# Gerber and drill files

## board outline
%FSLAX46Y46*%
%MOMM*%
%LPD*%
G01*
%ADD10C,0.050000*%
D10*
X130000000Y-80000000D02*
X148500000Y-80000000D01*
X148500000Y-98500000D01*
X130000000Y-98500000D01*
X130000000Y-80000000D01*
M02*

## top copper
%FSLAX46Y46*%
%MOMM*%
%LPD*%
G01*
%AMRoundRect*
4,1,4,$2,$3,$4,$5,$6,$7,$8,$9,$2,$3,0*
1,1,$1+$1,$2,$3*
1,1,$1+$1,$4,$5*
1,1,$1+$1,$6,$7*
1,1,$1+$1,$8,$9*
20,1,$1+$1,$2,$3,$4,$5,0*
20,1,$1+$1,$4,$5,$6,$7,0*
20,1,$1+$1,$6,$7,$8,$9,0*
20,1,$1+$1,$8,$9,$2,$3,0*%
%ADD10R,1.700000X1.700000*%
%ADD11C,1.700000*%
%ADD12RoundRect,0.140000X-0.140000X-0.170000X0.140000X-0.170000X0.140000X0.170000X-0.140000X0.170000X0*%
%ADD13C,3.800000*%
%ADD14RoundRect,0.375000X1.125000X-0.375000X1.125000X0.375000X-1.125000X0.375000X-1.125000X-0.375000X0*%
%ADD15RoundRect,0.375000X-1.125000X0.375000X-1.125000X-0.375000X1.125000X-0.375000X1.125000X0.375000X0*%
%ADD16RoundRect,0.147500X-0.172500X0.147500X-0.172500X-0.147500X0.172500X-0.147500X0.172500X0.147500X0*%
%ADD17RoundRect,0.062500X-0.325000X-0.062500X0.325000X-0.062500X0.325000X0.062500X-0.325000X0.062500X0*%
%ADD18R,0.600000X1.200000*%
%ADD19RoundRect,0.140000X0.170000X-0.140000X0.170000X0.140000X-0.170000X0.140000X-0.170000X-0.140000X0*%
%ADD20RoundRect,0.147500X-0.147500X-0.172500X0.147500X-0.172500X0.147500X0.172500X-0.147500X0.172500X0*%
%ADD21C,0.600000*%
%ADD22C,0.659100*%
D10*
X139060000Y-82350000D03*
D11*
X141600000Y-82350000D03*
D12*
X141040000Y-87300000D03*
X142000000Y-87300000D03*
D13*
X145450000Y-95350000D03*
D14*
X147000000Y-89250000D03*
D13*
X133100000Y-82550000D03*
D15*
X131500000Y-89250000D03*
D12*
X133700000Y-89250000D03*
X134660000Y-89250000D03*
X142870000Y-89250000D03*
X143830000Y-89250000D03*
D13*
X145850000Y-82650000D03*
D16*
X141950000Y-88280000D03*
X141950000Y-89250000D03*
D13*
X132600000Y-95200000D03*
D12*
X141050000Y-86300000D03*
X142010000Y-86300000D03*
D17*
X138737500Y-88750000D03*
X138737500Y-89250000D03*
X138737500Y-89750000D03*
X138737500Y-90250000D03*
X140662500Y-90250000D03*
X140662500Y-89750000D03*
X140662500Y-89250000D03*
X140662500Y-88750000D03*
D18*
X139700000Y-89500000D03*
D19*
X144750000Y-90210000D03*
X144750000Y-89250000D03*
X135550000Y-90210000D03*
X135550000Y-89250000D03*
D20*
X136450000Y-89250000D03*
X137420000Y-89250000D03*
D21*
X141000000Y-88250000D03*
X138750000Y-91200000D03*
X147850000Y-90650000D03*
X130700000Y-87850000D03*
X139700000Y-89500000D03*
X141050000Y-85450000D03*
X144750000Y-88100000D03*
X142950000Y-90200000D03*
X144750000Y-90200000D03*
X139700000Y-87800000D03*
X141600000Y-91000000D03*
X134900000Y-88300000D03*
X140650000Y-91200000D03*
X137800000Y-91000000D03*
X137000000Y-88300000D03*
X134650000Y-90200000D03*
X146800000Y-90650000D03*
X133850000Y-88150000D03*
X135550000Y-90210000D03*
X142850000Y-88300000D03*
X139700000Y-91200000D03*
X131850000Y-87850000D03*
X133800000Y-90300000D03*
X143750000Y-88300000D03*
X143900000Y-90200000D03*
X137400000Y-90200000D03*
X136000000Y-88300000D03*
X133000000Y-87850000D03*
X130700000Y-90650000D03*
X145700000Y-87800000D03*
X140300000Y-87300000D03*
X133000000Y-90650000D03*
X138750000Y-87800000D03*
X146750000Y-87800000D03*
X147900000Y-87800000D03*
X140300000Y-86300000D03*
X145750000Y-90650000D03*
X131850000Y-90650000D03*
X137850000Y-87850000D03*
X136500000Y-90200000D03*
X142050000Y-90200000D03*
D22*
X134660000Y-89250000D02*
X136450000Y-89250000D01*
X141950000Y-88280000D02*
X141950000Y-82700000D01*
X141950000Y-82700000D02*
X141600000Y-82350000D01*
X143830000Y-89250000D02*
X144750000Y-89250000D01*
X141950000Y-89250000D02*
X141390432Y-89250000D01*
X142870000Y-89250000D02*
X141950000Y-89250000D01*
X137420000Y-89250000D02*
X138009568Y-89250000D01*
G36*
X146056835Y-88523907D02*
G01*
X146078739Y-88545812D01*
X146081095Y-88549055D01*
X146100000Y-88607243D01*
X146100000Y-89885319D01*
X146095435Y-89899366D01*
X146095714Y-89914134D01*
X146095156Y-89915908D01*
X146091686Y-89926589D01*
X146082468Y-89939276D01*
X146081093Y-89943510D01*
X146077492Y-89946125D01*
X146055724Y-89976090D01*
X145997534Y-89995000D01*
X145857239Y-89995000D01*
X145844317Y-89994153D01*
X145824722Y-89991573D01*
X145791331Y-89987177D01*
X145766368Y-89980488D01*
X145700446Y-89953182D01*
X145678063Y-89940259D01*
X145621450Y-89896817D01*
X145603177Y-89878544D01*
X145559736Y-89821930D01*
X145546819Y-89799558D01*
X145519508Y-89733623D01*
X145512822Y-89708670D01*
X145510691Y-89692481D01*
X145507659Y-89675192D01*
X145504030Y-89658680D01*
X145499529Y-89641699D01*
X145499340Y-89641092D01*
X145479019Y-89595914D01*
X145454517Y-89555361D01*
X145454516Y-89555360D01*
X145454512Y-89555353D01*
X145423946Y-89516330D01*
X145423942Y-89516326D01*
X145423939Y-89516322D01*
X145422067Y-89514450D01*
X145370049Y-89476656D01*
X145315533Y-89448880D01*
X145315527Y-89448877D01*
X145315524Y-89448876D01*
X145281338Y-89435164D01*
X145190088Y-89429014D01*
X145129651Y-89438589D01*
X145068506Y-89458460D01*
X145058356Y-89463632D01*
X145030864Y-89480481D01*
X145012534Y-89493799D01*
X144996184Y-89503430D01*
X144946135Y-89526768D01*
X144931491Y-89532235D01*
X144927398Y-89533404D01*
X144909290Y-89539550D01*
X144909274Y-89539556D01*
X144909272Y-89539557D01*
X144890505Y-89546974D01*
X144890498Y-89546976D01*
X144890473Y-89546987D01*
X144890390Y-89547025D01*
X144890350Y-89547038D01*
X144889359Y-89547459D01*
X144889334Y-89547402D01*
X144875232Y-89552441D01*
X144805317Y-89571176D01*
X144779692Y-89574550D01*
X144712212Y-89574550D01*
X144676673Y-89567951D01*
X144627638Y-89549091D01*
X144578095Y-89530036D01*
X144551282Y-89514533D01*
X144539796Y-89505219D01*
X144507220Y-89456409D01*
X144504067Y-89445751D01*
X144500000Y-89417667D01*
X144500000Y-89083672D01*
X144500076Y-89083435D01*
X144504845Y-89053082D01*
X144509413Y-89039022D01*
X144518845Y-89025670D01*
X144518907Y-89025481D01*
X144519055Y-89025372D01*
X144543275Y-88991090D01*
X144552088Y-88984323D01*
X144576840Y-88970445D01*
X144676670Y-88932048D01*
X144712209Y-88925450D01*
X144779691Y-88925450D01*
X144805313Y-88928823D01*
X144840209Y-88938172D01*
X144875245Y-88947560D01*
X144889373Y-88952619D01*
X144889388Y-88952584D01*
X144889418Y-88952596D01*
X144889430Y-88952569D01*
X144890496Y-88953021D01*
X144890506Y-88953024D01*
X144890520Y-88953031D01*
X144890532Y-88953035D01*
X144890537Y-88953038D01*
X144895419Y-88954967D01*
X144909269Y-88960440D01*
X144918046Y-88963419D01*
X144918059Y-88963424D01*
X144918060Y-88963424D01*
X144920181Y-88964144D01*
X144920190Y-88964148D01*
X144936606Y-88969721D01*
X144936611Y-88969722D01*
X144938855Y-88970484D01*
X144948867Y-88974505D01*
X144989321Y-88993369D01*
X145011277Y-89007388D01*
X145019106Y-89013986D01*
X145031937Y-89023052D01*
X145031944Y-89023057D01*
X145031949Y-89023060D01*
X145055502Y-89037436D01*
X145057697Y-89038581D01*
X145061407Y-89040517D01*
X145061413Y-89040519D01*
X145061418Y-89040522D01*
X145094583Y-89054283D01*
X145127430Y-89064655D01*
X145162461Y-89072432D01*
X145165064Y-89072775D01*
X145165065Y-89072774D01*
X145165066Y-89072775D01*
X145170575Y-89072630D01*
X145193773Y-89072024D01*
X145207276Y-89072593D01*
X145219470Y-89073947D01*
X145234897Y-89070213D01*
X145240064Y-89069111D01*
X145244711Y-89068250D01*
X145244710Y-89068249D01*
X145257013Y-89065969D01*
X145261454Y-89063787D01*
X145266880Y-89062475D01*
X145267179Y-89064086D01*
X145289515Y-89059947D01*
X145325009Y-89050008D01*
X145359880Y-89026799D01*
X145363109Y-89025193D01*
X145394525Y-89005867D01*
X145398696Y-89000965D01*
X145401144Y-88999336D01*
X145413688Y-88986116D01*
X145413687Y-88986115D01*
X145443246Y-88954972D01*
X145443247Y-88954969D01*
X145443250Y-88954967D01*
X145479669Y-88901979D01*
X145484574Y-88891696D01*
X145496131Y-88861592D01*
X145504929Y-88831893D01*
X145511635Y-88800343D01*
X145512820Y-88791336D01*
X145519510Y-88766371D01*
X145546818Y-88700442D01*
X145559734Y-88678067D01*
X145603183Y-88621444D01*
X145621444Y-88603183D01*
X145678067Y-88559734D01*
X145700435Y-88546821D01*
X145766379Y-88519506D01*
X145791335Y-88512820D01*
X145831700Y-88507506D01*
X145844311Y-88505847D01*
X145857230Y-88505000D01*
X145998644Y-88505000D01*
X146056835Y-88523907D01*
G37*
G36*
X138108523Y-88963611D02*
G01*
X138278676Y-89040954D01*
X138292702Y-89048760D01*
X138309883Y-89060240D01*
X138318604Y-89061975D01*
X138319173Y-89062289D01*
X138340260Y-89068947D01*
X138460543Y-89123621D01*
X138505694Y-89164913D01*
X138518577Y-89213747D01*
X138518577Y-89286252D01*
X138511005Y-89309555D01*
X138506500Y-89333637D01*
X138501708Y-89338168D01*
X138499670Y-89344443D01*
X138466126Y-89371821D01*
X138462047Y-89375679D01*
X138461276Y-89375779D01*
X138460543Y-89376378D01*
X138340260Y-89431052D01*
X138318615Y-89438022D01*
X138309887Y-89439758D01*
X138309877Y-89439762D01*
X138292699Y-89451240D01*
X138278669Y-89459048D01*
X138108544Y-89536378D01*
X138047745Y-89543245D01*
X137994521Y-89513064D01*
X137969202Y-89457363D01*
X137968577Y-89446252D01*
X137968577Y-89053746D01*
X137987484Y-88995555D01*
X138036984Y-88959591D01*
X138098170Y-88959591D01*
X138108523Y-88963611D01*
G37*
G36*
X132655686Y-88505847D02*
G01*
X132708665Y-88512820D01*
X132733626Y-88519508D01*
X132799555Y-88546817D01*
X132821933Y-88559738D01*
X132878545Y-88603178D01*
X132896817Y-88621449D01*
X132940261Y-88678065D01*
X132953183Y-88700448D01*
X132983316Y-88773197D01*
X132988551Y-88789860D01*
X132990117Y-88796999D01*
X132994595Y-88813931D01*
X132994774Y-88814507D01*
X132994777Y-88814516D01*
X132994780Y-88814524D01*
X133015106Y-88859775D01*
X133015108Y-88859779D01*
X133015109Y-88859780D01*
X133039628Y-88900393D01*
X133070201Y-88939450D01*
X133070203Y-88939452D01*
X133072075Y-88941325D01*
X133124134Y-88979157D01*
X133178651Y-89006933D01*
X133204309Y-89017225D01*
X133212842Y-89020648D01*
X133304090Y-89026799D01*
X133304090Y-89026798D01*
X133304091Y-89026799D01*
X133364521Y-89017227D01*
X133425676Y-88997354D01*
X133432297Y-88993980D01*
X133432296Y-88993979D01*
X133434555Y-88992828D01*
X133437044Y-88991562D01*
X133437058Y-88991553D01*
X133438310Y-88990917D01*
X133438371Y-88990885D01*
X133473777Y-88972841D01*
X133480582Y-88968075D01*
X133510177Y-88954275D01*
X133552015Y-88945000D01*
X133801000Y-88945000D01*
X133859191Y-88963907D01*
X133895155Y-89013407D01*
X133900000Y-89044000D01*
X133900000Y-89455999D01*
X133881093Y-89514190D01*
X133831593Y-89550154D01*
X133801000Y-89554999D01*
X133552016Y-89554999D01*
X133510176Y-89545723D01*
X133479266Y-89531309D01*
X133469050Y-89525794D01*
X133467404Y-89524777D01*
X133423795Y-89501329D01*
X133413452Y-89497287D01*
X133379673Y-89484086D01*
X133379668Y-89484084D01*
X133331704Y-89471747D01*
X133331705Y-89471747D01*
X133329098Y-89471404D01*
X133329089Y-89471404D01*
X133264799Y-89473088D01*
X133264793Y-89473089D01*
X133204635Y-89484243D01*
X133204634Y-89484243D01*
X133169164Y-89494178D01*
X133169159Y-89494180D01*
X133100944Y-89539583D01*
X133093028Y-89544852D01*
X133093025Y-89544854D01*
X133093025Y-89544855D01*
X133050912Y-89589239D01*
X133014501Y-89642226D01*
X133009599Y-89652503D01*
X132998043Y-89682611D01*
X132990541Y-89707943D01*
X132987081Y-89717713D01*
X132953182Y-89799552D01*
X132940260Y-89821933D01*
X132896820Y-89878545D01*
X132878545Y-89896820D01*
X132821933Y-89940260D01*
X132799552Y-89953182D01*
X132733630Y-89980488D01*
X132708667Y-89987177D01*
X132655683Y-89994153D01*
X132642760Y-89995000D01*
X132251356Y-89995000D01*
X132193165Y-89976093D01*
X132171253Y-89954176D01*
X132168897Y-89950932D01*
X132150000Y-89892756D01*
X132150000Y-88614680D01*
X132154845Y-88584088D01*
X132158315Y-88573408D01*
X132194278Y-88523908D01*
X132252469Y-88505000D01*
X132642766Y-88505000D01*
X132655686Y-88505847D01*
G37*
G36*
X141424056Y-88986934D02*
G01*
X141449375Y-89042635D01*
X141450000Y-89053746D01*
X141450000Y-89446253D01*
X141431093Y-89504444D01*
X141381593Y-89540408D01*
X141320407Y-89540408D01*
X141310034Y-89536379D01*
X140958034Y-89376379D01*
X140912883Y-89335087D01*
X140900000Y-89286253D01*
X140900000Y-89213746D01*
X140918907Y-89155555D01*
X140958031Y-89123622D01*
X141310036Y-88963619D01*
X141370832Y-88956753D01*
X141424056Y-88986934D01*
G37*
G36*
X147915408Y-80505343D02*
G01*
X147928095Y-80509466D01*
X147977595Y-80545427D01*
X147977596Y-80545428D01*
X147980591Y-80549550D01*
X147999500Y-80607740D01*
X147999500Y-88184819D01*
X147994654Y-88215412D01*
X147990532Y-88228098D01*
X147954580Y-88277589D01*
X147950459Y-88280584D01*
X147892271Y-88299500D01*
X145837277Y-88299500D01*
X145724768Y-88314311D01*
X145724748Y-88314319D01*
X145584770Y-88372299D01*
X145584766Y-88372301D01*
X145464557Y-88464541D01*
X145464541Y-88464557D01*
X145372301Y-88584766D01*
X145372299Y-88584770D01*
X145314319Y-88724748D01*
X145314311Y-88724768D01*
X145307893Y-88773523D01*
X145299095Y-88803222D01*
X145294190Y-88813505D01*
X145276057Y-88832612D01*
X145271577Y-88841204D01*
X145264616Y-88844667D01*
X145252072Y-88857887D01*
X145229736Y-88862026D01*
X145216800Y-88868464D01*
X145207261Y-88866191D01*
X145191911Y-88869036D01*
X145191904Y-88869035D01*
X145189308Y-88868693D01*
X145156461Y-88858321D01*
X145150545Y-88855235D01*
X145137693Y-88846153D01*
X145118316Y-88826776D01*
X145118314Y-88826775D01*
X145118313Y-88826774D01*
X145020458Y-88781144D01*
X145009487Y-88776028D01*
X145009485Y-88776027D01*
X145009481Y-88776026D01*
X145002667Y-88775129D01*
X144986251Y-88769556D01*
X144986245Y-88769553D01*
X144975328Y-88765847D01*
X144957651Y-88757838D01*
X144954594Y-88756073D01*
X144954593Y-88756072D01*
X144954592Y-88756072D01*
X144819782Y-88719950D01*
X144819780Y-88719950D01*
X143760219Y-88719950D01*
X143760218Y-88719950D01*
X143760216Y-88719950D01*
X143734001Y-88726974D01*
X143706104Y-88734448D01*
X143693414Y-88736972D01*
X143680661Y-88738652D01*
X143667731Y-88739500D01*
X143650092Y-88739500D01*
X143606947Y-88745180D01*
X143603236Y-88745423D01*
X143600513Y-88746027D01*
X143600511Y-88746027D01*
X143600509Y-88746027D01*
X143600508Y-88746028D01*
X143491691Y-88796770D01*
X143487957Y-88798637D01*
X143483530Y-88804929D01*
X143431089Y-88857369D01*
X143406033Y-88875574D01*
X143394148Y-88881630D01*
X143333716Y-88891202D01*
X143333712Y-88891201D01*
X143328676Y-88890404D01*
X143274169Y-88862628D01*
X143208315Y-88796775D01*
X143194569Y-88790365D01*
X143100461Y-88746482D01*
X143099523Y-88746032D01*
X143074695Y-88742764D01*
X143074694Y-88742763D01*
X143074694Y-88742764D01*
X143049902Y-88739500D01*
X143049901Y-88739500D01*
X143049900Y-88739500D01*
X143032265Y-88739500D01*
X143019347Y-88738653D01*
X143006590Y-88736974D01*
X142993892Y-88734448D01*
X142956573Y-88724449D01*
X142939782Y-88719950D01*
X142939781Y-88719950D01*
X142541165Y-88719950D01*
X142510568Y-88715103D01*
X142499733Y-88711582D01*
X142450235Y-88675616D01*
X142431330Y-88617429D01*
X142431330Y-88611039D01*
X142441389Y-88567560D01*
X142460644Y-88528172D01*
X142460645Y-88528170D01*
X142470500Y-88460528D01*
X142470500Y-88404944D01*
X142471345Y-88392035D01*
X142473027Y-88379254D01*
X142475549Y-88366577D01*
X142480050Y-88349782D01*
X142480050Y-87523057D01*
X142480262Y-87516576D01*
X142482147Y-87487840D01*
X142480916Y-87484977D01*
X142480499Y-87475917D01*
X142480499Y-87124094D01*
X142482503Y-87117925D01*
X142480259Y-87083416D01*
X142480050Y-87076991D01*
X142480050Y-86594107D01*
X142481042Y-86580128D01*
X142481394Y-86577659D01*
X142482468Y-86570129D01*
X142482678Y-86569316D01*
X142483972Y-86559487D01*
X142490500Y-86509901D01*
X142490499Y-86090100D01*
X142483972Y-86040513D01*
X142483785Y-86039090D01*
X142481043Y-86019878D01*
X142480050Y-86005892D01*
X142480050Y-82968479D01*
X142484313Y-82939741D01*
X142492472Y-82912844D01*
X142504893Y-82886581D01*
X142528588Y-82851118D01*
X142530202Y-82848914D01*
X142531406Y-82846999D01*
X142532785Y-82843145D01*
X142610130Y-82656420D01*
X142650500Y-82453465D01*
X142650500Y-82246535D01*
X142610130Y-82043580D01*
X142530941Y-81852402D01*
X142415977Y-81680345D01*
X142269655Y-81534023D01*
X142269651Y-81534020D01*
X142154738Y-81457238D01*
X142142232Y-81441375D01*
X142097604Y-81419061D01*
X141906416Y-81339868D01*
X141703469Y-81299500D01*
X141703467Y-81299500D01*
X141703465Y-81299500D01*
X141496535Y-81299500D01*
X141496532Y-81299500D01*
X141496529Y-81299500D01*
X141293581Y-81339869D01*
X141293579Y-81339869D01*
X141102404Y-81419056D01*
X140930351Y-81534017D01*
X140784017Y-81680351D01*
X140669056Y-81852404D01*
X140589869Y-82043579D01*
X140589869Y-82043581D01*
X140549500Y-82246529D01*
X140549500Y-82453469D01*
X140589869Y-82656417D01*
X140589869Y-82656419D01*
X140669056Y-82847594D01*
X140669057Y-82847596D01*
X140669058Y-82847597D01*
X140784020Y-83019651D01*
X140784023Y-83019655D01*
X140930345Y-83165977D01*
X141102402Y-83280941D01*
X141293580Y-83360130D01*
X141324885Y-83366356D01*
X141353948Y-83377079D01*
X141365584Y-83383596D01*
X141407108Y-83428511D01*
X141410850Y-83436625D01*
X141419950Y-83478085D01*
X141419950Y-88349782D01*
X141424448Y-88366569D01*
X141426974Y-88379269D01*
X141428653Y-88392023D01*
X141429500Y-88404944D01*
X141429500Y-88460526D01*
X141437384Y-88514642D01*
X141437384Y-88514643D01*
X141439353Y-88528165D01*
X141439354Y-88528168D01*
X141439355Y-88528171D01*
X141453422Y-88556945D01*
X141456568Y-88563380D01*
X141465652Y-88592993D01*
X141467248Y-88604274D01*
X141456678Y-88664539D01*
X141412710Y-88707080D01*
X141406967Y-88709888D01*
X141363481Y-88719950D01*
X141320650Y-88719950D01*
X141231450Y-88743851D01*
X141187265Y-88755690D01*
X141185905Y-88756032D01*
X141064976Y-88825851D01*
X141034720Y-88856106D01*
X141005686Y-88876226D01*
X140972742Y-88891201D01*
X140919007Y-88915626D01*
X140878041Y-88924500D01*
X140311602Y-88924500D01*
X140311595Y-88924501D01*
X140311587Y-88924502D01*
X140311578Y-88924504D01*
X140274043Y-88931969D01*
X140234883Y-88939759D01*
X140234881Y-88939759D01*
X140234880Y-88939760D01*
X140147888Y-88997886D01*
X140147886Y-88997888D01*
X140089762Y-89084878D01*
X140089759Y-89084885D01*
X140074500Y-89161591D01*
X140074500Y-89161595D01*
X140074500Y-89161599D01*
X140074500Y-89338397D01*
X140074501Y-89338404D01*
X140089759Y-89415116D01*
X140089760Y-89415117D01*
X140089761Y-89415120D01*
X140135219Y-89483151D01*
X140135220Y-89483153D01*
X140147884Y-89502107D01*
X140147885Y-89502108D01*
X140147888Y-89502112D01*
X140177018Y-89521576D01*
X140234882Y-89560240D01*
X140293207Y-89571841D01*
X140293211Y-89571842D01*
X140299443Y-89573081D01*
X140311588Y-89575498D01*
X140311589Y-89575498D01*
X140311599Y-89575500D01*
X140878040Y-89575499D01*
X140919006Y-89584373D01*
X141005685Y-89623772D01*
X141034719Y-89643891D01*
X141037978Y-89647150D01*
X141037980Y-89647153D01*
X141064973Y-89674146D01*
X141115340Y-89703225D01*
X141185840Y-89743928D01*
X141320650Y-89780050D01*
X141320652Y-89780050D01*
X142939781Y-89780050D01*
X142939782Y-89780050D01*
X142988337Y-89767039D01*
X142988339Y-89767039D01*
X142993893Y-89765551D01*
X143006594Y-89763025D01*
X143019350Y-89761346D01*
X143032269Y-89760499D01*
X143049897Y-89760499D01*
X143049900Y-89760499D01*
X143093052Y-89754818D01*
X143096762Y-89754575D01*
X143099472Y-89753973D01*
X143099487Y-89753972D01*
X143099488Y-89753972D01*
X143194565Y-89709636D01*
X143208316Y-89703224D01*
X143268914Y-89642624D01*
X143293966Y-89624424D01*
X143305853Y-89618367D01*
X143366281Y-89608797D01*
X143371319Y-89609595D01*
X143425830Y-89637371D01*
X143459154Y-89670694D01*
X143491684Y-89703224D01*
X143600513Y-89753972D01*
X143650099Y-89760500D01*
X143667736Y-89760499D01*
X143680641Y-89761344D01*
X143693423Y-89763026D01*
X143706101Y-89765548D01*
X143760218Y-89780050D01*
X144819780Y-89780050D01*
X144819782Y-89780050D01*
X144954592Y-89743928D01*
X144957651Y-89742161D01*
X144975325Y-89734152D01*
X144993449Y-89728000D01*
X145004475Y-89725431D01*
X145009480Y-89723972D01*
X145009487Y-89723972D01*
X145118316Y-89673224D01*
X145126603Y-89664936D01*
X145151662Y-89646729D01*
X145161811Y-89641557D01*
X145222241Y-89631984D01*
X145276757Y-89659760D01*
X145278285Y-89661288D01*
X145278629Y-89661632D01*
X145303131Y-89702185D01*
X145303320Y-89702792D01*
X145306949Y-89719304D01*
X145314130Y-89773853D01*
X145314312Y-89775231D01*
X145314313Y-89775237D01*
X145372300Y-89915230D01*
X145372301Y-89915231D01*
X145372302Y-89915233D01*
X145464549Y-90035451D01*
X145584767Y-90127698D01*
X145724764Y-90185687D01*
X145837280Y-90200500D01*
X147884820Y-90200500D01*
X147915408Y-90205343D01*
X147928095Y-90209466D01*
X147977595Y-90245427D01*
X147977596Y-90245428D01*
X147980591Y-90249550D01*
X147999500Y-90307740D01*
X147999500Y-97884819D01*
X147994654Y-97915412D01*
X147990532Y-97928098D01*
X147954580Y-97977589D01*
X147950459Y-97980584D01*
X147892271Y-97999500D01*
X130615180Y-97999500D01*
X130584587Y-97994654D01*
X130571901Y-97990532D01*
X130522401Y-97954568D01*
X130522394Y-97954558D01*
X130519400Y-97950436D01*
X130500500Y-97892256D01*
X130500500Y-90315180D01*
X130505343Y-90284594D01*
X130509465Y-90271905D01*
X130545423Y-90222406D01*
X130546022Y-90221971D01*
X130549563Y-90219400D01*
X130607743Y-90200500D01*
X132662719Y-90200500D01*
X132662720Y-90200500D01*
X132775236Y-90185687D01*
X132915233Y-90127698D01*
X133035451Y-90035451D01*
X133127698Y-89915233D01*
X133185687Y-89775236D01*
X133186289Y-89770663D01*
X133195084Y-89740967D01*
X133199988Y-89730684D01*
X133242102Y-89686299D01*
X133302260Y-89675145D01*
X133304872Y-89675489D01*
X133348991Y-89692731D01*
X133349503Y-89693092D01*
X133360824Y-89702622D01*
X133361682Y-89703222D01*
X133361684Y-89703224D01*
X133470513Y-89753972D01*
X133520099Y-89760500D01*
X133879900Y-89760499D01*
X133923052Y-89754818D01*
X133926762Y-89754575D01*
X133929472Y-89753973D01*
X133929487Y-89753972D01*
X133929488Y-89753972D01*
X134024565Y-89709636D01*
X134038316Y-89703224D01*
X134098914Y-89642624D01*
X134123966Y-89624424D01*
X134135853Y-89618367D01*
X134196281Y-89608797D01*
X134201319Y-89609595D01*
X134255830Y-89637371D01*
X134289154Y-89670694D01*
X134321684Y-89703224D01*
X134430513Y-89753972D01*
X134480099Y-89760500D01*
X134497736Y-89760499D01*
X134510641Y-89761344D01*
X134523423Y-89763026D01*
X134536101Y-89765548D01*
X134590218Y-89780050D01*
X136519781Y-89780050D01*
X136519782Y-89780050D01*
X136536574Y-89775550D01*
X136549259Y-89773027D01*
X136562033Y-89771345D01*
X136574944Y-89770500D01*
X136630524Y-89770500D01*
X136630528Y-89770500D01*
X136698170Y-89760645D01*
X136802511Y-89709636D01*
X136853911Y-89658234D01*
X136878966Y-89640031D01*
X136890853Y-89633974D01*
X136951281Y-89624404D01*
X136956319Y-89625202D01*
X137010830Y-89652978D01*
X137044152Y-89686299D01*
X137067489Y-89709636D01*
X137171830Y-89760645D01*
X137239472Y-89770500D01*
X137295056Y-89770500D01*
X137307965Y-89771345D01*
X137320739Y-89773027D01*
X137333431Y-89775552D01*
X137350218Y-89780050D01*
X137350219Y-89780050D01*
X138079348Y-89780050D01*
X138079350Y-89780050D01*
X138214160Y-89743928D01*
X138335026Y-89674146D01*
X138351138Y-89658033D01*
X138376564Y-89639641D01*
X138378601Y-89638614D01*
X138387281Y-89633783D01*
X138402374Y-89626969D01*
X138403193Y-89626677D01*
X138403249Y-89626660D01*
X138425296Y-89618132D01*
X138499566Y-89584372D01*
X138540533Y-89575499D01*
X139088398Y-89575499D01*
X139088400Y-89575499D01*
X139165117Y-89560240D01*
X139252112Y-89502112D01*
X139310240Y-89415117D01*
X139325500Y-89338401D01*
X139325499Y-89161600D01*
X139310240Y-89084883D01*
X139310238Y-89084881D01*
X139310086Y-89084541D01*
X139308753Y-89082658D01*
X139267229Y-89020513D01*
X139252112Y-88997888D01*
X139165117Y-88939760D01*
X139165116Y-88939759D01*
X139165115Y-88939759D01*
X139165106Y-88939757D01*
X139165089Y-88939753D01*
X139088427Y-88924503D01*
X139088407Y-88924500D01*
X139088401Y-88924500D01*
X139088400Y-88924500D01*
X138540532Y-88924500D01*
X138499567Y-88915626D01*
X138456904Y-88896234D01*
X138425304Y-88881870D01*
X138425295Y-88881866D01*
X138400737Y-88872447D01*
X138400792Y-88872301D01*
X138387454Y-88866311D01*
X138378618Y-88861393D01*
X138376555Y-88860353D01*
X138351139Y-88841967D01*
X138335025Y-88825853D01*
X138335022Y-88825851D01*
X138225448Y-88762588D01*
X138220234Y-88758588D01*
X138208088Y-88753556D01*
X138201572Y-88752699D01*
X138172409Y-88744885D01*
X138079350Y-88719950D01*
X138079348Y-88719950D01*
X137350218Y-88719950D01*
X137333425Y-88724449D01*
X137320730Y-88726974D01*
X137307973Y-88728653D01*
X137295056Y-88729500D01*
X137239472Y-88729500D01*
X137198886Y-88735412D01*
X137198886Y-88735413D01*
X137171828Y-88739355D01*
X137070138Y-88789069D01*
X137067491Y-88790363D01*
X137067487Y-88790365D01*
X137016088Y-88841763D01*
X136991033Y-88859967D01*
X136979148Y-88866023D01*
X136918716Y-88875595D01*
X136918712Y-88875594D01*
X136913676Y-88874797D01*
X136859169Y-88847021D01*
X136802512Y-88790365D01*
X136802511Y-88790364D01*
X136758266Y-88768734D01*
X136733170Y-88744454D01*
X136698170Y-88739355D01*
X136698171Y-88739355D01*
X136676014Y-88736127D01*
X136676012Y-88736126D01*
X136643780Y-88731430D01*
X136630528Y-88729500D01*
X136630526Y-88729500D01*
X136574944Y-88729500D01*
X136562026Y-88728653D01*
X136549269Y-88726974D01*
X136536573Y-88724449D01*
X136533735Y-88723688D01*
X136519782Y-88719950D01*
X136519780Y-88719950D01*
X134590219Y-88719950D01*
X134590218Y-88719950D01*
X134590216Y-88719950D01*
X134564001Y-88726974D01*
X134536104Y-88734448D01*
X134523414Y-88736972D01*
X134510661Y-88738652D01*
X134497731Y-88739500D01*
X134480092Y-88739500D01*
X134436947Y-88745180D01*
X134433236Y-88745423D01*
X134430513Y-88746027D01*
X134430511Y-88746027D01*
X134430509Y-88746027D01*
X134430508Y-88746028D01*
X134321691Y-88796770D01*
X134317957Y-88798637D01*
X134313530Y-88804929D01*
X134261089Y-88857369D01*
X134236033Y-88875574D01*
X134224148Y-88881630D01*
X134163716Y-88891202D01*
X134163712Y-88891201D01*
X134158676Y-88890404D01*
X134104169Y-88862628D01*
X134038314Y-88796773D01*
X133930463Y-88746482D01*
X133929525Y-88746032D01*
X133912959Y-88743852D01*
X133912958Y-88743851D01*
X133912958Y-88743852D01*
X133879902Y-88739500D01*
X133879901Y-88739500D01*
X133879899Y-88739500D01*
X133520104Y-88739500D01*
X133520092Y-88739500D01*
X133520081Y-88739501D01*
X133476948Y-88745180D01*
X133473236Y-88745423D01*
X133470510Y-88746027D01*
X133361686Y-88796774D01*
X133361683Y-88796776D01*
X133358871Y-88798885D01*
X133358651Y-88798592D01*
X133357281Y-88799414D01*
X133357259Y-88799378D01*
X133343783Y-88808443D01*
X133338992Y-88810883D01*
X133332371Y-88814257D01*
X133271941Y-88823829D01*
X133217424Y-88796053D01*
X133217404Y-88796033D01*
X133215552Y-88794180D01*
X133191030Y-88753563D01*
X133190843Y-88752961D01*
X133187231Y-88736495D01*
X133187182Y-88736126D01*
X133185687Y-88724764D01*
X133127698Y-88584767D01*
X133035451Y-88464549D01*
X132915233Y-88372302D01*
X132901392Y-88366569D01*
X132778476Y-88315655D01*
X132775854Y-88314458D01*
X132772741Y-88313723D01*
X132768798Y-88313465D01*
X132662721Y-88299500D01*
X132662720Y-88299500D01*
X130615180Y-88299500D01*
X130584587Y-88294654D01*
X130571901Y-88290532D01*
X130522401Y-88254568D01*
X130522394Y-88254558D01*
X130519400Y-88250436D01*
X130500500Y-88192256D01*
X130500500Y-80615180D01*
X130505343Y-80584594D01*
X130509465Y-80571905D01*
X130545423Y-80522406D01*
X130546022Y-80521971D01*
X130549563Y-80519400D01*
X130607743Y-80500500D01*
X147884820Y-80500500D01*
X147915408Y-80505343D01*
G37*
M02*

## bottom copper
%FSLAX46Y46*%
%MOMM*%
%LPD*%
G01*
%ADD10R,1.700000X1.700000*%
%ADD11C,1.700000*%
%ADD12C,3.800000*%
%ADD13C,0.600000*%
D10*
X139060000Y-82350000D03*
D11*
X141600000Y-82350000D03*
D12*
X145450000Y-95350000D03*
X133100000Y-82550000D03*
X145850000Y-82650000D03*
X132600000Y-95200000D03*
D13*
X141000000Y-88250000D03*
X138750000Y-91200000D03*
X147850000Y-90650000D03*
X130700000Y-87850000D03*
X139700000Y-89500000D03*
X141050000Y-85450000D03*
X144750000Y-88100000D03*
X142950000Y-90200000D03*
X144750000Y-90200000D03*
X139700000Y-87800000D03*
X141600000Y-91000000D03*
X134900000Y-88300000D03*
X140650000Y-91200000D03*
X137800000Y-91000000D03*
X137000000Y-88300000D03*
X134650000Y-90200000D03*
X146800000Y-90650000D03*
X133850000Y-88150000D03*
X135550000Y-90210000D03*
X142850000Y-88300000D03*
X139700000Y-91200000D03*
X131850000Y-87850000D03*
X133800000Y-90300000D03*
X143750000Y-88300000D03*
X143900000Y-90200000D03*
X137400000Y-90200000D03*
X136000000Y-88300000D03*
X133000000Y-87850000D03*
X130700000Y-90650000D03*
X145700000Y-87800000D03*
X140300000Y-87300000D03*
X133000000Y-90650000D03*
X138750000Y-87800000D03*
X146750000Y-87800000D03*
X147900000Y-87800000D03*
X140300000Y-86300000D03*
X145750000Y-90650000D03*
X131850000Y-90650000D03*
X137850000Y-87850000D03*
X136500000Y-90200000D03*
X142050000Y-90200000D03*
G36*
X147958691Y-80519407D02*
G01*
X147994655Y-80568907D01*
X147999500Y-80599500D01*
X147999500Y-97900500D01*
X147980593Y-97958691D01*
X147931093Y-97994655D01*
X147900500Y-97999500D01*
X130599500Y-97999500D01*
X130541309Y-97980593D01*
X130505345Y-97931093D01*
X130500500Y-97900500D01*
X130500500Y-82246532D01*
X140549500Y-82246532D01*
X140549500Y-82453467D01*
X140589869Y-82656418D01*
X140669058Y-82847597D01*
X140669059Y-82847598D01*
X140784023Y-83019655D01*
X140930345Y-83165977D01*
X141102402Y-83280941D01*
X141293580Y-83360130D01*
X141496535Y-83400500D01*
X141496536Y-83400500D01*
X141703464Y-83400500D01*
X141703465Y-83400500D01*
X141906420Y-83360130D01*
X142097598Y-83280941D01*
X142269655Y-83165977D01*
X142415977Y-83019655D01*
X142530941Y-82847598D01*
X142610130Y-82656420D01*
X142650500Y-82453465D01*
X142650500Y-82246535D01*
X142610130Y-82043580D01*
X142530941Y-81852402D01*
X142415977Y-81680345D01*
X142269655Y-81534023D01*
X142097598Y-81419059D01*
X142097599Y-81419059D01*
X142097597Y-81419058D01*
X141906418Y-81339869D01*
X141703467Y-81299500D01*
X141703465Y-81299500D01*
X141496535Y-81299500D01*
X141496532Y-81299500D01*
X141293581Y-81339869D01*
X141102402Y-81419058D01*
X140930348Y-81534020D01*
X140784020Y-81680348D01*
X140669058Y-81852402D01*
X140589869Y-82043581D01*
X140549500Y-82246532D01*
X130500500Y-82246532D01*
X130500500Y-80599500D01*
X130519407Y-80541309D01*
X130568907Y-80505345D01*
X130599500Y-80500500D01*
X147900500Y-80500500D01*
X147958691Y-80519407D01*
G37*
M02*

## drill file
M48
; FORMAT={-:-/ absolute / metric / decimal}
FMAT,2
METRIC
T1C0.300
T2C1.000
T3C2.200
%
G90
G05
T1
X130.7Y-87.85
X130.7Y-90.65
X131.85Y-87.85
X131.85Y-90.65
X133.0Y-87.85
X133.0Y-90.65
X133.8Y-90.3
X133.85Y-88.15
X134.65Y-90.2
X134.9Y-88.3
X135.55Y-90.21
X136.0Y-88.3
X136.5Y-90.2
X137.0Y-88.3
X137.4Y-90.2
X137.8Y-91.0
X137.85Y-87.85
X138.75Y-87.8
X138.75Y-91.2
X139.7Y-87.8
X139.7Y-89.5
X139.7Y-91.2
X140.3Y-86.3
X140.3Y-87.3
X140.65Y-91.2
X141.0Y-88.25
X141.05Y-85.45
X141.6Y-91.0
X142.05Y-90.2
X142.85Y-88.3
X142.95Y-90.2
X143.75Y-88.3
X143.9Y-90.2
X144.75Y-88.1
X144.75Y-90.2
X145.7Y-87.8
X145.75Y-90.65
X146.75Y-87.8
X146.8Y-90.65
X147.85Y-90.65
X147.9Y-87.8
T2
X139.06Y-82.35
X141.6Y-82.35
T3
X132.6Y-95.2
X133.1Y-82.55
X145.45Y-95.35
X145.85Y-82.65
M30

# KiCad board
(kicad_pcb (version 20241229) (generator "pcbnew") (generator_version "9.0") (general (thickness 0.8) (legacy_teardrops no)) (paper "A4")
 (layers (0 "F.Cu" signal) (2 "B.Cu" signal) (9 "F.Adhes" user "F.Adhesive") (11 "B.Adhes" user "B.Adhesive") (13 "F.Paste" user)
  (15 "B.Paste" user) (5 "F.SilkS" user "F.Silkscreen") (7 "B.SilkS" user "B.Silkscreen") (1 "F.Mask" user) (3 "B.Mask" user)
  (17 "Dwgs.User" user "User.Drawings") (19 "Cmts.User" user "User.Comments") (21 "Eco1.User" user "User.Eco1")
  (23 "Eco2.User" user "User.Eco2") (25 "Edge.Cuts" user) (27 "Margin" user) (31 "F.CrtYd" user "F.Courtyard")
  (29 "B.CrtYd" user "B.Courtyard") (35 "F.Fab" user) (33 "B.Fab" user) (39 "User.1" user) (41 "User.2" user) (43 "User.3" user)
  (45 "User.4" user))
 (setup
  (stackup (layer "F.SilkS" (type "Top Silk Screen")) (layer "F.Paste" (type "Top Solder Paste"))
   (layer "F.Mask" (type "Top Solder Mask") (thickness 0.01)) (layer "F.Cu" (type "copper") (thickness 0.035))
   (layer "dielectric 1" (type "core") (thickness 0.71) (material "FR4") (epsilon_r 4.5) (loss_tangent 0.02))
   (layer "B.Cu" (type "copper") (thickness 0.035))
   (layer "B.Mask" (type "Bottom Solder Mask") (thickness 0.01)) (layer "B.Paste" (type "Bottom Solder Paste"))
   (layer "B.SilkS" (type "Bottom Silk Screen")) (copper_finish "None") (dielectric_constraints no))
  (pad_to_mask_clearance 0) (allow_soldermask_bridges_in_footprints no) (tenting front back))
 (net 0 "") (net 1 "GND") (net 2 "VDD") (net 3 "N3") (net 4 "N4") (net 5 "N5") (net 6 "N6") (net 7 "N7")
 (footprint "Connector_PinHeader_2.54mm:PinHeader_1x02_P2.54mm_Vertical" (layer "F.Cu") (at 139.06 82.35 90)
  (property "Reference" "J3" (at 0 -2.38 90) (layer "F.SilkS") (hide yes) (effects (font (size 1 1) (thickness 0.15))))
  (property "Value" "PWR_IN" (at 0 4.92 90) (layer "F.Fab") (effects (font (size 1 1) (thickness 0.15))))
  (pad "1" thru_hole rect (at 0 0 90) (size 1.7 1.7) (drill 1) (layers "*.Cu" "*.Mask") (remove_unused_layers no) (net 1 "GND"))
  (pad "2" thru_hole circle (at 0 2.54 90) (size 1.7 1.7) (drill 1) (layers "*.Cu" "*.Mask") (remove_unused_layers no) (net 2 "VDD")))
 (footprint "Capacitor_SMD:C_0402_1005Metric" (layer "F.Cu") (at 141.52 87.3)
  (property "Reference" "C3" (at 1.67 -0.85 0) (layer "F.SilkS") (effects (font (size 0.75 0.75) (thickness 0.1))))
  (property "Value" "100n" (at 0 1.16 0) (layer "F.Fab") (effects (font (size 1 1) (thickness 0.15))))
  (pad "1" smd roundrect (at -0.48 0) (size 0.56 0.62) (layers "F.Cu" "F.Mask" "F.Paste") (roundrect_rratio 0.25) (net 1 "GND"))
  (pad "2" smd roundrect (at 0.48 0) (size 0.56 0.62) (layers "F.Cu" "F.Mask" "F.Paste") (roundrect_rratio 0.25) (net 2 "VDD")))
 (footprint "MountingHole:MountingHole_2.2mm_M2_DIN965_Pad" (layer "F.Cu") (at 145.45 95.35)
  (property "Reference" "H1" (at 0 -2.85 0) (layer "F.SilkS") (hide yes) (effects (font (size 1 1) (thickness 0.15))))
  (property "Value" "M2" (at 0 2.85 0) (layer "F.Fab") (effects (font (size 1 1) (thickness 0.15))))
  (pad "1" thru_hole circle (at 0 0) (size 3.8 3.8) (drill 2.2) (layers "*.Cu" "*.Mask") (remove_unused_layers no) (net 1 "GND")
   (zone_connect 2)))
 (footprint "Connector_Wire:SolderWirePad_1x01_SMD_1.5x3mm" (layer "F.Cu") (at 147 89.25 90)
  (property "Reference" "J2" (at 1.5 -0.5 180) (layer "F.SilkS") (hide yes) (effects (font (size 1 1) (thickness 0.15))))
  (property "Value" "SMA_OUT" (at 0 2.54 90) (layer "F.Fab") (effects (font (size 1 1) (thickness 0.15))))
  (pad "1" smd roundrect (at 0 0 90) (size 1.5 3) (layers "F.Cu" "F.Mask") (roundrect_rratio 0.25) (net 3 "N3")))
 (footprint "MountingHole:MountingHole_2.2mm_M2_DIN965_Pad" (layer "F.Cu") (at 133.1 82.55)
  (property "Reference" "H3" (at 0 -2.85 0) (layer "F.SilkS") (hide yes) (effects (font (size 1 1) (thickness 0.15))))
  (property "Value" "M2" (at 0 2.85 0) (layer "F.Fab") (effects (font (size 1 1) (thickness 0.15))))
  (pad "1" thru_hole circle (at 0 0) (size 3.8 3.8) (drill 2.2) (layers "*.Cu" "*.Mask") (remove_unused_layers no) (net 1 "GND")
   (zone_connect 2)))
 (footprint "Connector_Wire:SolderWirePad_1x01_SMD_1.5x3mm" (layer "F.Cu") (at 131.5 89.25 -90)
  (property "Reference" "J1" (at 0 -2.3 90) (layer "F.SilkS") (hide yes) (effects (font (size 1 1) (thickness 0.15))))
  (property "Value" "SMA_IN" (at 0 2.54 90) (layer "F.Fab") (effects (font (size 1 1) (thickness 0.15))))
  (pad "1" smd roundrect (at 0 0 270) (size 1.5 3) (layers "F.Cu" "F.Mask") (roundrect_rratio 0.25) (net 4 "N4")))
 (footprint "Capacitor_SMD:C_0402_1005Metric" (layer "F.Cu") (at 134.18 89.25)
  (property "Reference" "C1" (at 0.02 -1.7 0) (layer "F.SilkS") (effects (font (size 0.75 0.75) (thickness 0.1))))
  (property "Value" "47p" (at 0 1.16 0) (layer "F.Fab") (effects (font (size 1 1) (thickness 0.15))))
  (pad "1" smd roundrect (at -0.48 0) (size 0.56 0.62) (layers "F.Cu" "F.Mask" "F.Paste") (roundrect_rratio 0.25) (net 4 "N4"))
  (pad "2" smd roundrect (at 0.48 0) (size 0.56 0.62) (layers "F.Cu" "F.Mask" "F.Paste") (roundrect_rratio 0.25) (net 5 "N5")))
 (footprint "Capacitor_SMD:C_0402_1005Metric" (layer "F.Cu") (at 143.35 89.25)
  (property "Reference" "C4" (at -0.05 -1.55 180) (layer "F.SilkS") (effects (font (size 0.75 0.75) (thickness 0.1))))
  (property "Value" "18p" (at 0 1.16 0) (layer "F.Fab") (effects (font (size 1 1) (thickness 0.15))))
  (pad "1" smd roundrect (at -0.48 0) (size 0.56 0.62) (layers "F.Cu" "F.Mask" "F.Paste") (roundrect_rratio 0.25) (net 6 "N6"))
  (pad "2" smd roundrect (at 0.48 0) (size 0.56 0.62) (layers "F.Cu" "F.Mask" "F.Paste") (roundrect_rratio 0.25) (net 3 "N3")))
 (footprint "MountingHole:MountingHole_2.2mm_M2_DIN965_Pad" (layer "F.Cu") (at 145.85 82.65)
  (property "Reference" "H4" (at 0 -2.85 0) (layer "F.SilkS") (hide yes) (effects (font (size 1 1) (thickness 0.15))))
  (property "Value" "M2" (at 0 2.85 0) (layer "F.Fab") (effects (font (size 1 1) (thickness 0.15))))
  (pad "1" thru_hole circle (at 0 0) (size 3.8 3.8) (drill 2.2) (layers "*.Cu" "*.Mask") (remove_unused_layers no) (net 1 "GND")
   (zone_connect 2)))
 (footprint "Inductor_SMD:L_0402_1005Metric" (layer "F.Cu") (at 141.95 88.765 -90)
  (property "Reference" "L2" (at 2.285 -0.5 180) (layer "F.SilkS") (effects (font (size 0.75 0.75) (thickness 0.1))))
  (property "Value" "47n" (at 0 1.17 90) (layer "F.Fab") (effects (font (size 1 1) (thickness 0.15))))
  (pad "1" smd roundrect (at -0.485 0 270) (size 0.59 0.64) (layers "F.Cu" "F.Mask" "F.Paste") (roundrect_rratio 0.25) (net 2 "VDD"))
  (pad "2" smd roundrect (at 0.485 0 270) (size 0.59 0.64) (layers "F.Cu" "F.Mask" "F.Paste") (roundrect_rratio 0.25) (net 6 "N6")))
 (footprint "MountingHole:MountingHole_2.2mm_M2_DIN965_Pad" (layer "F.Cu") (at 132.6 95.2)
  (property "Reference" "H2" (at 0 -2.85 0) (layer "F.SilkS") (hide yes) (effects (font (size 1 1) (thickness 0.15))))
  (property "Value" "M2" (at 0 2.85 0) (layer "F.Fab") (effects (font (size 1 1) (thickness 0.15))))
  (pad "1" thru_hole circle (at 0 0) (size 3.8 3.8) (drill 2.2) (layers "*.Cu" "*.Mask") (remove_unused_layers no) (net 1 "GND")
   (zone_connect 2)))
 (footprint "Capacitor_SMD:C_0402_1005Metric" (layer "F.Cu") (at 141.53 86.3)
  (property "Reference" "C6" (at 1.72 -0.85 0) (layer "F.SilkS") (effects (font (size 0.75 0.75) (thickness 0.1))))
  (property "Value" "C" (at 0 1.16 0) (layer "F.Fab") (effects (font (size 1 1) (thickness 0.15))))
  (pad "1" smd roundrect (at -0.48 0) (size 0.56 0.62) (layers "F.Cu" "F.Mask" "F.Paste") (roundrect_rratio 0.25) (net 1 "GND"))
  (pad "2" smd roundrect (at 0.48 0) (size 0.56 0.62) (layers "F.Cu" "F.Mask" "F.Paste") (roundrect_rratio 0.25) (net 2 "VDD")))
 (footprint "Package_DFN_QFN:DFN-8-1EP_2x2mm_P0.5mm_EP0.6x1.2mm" (layer "F.Cu") (at 139.7 89.5)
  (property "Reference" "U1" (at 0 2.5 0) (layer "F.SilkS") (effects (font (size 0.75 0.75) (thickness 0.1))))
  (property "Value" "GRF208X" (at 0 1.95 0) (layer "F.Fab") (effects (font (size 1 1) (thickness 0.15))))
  (pad "" smd roundrect (at -0.15 -0.3) (size 0.24 0.48) (layers "F.Paste") (roundrect_rratio 0.25))
  (pad "" smd roundrect (at -0.15 0.3) (size 0.24 0.48) (layers "F.Paste") (roundrect_rratio 0.25))
  (pad "" smd roundrect (at 0.15 -0.3) (size 0.24 0.48) (layers "F.Paste") (roundrect_rratio 0.25))
  (pad "" smd roundrect (at 0.15 0.3) (size 0.24 0.48) (layers "F.Paste") (roundrect_rratio 0.25))
  (pad "1" smd roundrect (at -0.9625 -0.75) (size 0.775 0.25) (layers "F.Cu" "F.Mask" "F.Paste") (roundrect_rratio 0.25) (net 1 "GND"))
  (pad "2" smd roundrect (at -0.9625 -0.25) (size 0.775 0.25) (layers "F.Cu" "F.Mask" "F.Paste") (roundrect_rratio 0.25) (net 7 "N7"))
  (pad "3" smd roundrect (at -0.9625 0.25) (size 0.775 0.25) (layers "F.Cu" "F.Mask" "F.Paste") (roundrect_rratio 0.25) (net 1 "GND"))
  (pad "4" smd roundrect (at -0.9625 0.75) (size 0.775 0.25) (layers "F.Cu" "F.Mask" "F.Paste") (roundrect_rratio 0.25) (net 1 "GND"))
  (pad "5" smd roundrect (at 0.9625 0.75) (size 0.775 0.25) (layers "F.Cu" "F.Mask" "F.Paste") (roundrect_rratio 0.25) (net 1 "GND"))
  (pad "6" smd roundrect (at 0.9625 0.25) (size 0.775 0.25) (layers "F.Cu" "F.Mask" "F.Paste") (roundrect_rratio 0.25) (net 1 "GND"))
  (pad "7" smd roundrect (at 0.9625 -0.25) (size 0.775 0.25) (layers "F.Cu" "F.Mask" "F.Paste") (roundrect_rratio 0.25) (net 6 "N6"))
  (pad "8" smd roundrect (at 0.9625 -0.75) (size 0.775 0.25) (layers "F.Cu" "F.Mask" "F.Paste") (roundrect_rratio 0.25) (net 1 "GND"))
  (pad "9" smd rect (at 0 0) (size 0.6 1.2) (layers "F.Cu" "F.Mask") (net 1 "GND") (zone_connect 2)))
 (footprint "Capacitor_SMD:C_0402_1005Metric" (layer "F.Cu") (at 144.75 89.73 90)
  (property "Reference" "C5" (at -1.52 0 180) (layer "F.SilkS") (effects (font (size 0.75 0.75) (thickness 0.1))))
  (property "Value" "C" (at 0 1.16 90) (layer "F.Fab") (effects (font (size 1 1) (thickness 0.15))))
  (pad "1" smd roundrect (at -0.48 0 90) (size 0.56 0.62) (layers "F.Cu" "F.Mask" "F.Paste") (roundrect_rratio 0.25) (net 1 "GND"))
  (pad "2" smd roundrect (at 0.48 0 90) (size 0.56 0.62) (layers "F.Cu" "F.Mask" "F.Paste") (roundrect_rratio 0.25) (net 3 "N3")))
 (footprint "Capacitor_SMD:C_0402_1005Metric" (layer "F.Cu") (at 135.55 89.73 90)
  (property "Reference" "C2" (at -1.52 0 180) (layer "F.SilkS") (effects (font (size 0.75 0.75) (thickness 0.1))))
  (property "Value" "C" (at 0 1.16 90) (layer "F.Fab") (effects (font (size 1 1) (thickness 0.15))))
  (pad "1" smd roundrect (at -0.48 0 90) (size 0.56 0.62) (layers "F.Cu" "F.Mask" "F.Paste") (roundrect_rratio 0.25) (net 1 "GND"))
  (pad "2" smd roundrect (at 0.48 0 90) (size 0.56 0.62) (layers "F.Cu" "F.Mask" "F.Paste") (roundrect_rratio 0.25) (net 5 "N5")))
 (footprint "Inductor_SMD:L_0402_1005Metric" (layer "F.Cu") (at 136.935 89.25)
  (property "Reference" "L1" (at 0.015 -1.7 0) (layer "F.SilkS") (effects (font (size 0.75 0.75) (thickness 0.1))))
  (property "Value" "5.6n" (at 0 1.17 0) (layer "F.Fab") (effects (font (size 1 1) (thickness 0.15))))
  (pad "1" smd roundrect (at -0.485 0) (size 0.59 0.64) (layers "F.Cu" "F.Mask" "F.Paste") (roundrect_rratio 0.25) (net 5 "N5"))
  (pad "2" smd roundrect (at 0.485 0) (size 0.59 0.64) (layers "F.Cu" "F.Mask" "F.Paste") (roundrect_rratio 0.25) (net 7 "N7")))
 (gr_rect (start 130 80) (end 148.5 98.5) (stroke (width 0.05) (type default)) (fill no) (layer "Edge.Cuts"))
 (via (at 141 88.25) (size 0.6) (drill 0.3) (layers "F.Cu" "B.Cu") (free yes) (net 1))
 (via (at 138.75 91.2) (size 0.6) (drill 0.3) (layers "F.Cu" "B.Cu") (free yes) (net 1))
 (via (at 147.85 90.65) (size 0.6) (drill 0.3) (layers "F.Cu" "B.Cu") (free yes) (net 1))
 (via (at 130.7 87.85) (size 0.6) (drill 0.3) (layers "F.Cu" "B.Cu") (free yes) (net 1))
 (via (at 139.7 89.5) (size 0.6) (drill 0.3) (layers "F.Cu" "B.Cu") (free yes) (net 1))
 (via (at 141.05 85.45) (size 0.6) (drill 0.3) (layers "F.Cu" "B.Cu") (free yes) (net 1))
 (via (at 144.75 88.1) (size 0.6) (drill 0.3) (layers "F.Cu" "B.Cu") (free yes) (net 1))
 (via (at 142.95 90.2) (size 0.6) (drill 0.3) (layers "F.Cu" "B.Cu") (free yes) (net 1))
 (via (at 144.75 90.2) (size 0.6) (drill 0.3) (layers "F.Cu" "B.Cu") (free yes) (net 1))
 (via (at 139.7 87.8) (size 0.6) (drill 0.3) (layers "F.Cu" "B.Cu") (free yes) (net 1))
 (via (at 141.6 91) (size 0.6) (drill 0.3) (layers "F.Cu" "B.Cu") (free yes) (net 1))
 (via (at 134.9 88.3) (size 0.6) (drill 0.3) (layers "F.Cu" "B.Cu") (free yes) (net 1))
 (via (at 140.65 91.2) (size 0.6) (drill 0.3) (layers "F.Cu" "B.Cu") (free yes) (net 1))
 (via (at 137.8 91) (size 0.6) (drill 0.3) (layers "F.Cu" "B.Cu") (free yes) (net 1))
 (via (at 137 88.3) (size 0.6) (drill 0.3) (layers "F.Cu" "B.Cu") (free yes) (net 1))
 (via (at 134.65 90.2) (size 0.6) (drill 0.3) (layers "F.Cu" "B.Cu") (free yes) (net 1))
 (via (at 146.8 90.65) (size 0.6) (drill 0.3) (layers "F.Cu" "B.Cu") (free yes) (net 1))
 (via (at 133.85 88.15) (size 0.6) (drill 0.3) (layers "F.Cu" "B.Cu") (free yes) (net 1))
 (via (at 135.55 90.21) (size 0.6) (drill 0.3) (layers "F.Cu" "B.Cu") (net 1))
 (via (at 142.85 88.3) (size 0.6) (drill 0.3) (layers "F.Cu" "B.Cu") (free yes) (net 1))
 (via (at 139.7 91.2) (size 0.6) (drill 0.3) (layers "F.Cu" "B.Cu") (free yes) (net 1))
 (via (at 131.85 87.85) (size 0.6) (drill 0.3) (layers "F.Cu" "B.Cu") (free yes) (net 1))
 (via (at 133.8 90.3) (size 0.6) (drill 0.3) (layers "F.Cu" "B.Cu") (free yes) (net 1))
 (via (at 143.75 88.3) (size 0.6) (drill 0.3) (layers "F.Cu" "B.Cu") (free yes) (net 1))
 (via (at 143.9 90.2) (size 0.6) (drill 0.3) (layers "F.Cu" "B.Cu") (free yes) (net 1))
 (via (at 137.4 90.2) (size 0.6) (drill 0.3) (layers "F.Cu" "B.Cu") (free yes) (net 1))
 (via (at 136 88.3) (size 0.6) (drill 0.3) (layers "F.Cu" "B.Cu") (free yes) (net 1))
 (via (at 133 87.85) (size 0.6) (drill 0.3) (layers "F.Cu" "B.Cu") (free yes) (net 1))
 (via (at 130.7 90.65) (size 0.6) (drill 0.3) (layers "F.Cu" "B.Cu") (free yes) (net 1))
 (via (at 145.7 87.8) (size 0.6) (drill 0.3) (layers "F.Cu" "B.Cu") (free yes) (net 1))
 (via (at 140.3 87.3) (size 0.6) (drill 0.3) (layers "F.Cu" "B.Cu") (free yes) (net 1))
 (via (at 133 90.65) (size 0.6) (drill 0.3) (layers "F.Cu" "B.Cu") (free yes) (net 1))
 (via (at 138.75 87.8) (size 0.6) (drill 0.3) (layers "F.Cu" "B.Cu") (free yes) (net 1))
 (via (at 146.75 87.8) (size 0.6) (drill 0.3) (layers "F.Cu" "B.Cu") (free yes) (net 1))
 (via (at 147.9 87.8) (size 0.6) (drill 0.3) (layers "F.Cu" "B.Cu") (free yes) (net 1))
 (via (at 140.3 86.3) (size 0.6) (drill 0.3) (layers "F.Cu" "B.Cu") (free yes) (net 1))
 (via (at 145.75 90.65) (size 0.6) (drill 0.3) (layers "F.Cu" "B.Cu") (free yes) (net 1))
 (via (at 131.85 90.65) (size 0.6) (drill 0.3) (layers "F.Cu" "B.Cu") (free yes) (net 1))
 (via (at 137.85 87.85) (size 0.6) (drill 0.3) (layers "F.Cu" "B.Cu") (free yes) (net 1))
 (via (at 136.5 90.2) (size 0.6) (drill 0.3) (layers "F.Cu" "B.Cu") (free yes) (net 1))
 (via (at 142.05 90.2) (size 0.6) (drill 0.3) (layers "F.Cu" "B.Cu") (free yes) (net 1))
 (segment (start 134.66 89.25) (end 136.45 89.25) (width 0.6591) (layer "F.Cu") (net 5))
 (segment (start 141.95 88.28) (end 141.95 82.7) (width 0.6591) (layer "F.Cu") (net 2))
 (segment (start 141.95 82.7) (end 141.6 82.35) (width 0.6591) (layer "F.Cu") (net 2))
 (segment (start 143.83 89.25) (end 144.75 89.25) (width 0.6591) (layer "F.Cu") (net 3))
 (segment (start 141.95 89.25) (end 141.390432 89.25) (width 0.6591) (layer "F.Cu") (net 6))
 (segment (start 142.87 89.25) (end 141.95 89.25) (width 0.6591) (layer "F.Cu") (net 6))
 (segment (start 137.42 89.25) (end 138.009568 89.25) (width 0.6591) (layer "F.Cu") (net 7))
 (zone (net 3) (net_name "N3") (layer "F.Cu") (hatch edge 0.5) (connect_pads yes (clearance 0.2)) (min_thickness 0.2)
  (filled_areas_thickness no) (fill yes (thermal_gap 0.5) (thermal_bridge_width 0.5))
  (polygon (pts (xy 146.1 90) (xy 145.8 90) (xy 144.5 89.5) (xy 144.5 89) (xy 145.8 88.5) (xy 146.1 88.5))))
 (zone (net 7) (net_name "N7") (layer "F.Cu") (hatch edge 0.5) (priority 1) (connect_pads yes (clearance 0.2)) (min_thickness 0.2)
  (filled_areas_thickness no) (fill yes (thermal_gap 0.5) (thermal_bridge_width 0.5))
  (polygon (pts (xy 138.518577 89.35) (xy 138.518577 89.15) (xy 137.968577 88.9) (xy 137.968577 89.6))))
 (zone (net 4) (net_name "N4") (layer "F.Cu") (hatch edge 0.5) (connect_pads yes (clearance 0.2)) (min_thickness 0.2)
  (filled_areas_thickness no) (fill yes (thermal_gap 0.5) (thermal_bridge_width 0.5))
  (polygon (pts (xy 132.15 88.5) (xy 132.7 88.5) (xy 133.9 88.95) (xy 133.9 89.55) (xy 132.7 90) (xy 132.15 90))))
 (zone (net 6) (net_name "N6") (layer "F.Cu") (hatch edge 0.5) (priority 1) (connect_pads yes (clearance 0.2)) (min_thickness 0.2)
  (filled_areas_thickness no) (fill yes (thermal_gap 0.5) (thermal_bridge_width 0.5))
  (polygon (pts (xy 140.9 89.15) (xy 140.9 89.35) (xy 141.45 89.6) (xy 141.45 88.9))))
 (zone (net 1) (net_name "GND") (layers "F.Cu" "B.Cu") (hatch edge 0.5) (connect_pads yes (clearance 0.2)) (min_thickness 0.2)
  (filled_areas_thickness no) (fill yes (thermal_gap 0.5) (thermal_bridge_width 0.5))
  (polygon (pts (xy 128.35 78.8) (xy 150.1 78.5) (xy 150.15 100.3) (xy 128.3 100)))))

